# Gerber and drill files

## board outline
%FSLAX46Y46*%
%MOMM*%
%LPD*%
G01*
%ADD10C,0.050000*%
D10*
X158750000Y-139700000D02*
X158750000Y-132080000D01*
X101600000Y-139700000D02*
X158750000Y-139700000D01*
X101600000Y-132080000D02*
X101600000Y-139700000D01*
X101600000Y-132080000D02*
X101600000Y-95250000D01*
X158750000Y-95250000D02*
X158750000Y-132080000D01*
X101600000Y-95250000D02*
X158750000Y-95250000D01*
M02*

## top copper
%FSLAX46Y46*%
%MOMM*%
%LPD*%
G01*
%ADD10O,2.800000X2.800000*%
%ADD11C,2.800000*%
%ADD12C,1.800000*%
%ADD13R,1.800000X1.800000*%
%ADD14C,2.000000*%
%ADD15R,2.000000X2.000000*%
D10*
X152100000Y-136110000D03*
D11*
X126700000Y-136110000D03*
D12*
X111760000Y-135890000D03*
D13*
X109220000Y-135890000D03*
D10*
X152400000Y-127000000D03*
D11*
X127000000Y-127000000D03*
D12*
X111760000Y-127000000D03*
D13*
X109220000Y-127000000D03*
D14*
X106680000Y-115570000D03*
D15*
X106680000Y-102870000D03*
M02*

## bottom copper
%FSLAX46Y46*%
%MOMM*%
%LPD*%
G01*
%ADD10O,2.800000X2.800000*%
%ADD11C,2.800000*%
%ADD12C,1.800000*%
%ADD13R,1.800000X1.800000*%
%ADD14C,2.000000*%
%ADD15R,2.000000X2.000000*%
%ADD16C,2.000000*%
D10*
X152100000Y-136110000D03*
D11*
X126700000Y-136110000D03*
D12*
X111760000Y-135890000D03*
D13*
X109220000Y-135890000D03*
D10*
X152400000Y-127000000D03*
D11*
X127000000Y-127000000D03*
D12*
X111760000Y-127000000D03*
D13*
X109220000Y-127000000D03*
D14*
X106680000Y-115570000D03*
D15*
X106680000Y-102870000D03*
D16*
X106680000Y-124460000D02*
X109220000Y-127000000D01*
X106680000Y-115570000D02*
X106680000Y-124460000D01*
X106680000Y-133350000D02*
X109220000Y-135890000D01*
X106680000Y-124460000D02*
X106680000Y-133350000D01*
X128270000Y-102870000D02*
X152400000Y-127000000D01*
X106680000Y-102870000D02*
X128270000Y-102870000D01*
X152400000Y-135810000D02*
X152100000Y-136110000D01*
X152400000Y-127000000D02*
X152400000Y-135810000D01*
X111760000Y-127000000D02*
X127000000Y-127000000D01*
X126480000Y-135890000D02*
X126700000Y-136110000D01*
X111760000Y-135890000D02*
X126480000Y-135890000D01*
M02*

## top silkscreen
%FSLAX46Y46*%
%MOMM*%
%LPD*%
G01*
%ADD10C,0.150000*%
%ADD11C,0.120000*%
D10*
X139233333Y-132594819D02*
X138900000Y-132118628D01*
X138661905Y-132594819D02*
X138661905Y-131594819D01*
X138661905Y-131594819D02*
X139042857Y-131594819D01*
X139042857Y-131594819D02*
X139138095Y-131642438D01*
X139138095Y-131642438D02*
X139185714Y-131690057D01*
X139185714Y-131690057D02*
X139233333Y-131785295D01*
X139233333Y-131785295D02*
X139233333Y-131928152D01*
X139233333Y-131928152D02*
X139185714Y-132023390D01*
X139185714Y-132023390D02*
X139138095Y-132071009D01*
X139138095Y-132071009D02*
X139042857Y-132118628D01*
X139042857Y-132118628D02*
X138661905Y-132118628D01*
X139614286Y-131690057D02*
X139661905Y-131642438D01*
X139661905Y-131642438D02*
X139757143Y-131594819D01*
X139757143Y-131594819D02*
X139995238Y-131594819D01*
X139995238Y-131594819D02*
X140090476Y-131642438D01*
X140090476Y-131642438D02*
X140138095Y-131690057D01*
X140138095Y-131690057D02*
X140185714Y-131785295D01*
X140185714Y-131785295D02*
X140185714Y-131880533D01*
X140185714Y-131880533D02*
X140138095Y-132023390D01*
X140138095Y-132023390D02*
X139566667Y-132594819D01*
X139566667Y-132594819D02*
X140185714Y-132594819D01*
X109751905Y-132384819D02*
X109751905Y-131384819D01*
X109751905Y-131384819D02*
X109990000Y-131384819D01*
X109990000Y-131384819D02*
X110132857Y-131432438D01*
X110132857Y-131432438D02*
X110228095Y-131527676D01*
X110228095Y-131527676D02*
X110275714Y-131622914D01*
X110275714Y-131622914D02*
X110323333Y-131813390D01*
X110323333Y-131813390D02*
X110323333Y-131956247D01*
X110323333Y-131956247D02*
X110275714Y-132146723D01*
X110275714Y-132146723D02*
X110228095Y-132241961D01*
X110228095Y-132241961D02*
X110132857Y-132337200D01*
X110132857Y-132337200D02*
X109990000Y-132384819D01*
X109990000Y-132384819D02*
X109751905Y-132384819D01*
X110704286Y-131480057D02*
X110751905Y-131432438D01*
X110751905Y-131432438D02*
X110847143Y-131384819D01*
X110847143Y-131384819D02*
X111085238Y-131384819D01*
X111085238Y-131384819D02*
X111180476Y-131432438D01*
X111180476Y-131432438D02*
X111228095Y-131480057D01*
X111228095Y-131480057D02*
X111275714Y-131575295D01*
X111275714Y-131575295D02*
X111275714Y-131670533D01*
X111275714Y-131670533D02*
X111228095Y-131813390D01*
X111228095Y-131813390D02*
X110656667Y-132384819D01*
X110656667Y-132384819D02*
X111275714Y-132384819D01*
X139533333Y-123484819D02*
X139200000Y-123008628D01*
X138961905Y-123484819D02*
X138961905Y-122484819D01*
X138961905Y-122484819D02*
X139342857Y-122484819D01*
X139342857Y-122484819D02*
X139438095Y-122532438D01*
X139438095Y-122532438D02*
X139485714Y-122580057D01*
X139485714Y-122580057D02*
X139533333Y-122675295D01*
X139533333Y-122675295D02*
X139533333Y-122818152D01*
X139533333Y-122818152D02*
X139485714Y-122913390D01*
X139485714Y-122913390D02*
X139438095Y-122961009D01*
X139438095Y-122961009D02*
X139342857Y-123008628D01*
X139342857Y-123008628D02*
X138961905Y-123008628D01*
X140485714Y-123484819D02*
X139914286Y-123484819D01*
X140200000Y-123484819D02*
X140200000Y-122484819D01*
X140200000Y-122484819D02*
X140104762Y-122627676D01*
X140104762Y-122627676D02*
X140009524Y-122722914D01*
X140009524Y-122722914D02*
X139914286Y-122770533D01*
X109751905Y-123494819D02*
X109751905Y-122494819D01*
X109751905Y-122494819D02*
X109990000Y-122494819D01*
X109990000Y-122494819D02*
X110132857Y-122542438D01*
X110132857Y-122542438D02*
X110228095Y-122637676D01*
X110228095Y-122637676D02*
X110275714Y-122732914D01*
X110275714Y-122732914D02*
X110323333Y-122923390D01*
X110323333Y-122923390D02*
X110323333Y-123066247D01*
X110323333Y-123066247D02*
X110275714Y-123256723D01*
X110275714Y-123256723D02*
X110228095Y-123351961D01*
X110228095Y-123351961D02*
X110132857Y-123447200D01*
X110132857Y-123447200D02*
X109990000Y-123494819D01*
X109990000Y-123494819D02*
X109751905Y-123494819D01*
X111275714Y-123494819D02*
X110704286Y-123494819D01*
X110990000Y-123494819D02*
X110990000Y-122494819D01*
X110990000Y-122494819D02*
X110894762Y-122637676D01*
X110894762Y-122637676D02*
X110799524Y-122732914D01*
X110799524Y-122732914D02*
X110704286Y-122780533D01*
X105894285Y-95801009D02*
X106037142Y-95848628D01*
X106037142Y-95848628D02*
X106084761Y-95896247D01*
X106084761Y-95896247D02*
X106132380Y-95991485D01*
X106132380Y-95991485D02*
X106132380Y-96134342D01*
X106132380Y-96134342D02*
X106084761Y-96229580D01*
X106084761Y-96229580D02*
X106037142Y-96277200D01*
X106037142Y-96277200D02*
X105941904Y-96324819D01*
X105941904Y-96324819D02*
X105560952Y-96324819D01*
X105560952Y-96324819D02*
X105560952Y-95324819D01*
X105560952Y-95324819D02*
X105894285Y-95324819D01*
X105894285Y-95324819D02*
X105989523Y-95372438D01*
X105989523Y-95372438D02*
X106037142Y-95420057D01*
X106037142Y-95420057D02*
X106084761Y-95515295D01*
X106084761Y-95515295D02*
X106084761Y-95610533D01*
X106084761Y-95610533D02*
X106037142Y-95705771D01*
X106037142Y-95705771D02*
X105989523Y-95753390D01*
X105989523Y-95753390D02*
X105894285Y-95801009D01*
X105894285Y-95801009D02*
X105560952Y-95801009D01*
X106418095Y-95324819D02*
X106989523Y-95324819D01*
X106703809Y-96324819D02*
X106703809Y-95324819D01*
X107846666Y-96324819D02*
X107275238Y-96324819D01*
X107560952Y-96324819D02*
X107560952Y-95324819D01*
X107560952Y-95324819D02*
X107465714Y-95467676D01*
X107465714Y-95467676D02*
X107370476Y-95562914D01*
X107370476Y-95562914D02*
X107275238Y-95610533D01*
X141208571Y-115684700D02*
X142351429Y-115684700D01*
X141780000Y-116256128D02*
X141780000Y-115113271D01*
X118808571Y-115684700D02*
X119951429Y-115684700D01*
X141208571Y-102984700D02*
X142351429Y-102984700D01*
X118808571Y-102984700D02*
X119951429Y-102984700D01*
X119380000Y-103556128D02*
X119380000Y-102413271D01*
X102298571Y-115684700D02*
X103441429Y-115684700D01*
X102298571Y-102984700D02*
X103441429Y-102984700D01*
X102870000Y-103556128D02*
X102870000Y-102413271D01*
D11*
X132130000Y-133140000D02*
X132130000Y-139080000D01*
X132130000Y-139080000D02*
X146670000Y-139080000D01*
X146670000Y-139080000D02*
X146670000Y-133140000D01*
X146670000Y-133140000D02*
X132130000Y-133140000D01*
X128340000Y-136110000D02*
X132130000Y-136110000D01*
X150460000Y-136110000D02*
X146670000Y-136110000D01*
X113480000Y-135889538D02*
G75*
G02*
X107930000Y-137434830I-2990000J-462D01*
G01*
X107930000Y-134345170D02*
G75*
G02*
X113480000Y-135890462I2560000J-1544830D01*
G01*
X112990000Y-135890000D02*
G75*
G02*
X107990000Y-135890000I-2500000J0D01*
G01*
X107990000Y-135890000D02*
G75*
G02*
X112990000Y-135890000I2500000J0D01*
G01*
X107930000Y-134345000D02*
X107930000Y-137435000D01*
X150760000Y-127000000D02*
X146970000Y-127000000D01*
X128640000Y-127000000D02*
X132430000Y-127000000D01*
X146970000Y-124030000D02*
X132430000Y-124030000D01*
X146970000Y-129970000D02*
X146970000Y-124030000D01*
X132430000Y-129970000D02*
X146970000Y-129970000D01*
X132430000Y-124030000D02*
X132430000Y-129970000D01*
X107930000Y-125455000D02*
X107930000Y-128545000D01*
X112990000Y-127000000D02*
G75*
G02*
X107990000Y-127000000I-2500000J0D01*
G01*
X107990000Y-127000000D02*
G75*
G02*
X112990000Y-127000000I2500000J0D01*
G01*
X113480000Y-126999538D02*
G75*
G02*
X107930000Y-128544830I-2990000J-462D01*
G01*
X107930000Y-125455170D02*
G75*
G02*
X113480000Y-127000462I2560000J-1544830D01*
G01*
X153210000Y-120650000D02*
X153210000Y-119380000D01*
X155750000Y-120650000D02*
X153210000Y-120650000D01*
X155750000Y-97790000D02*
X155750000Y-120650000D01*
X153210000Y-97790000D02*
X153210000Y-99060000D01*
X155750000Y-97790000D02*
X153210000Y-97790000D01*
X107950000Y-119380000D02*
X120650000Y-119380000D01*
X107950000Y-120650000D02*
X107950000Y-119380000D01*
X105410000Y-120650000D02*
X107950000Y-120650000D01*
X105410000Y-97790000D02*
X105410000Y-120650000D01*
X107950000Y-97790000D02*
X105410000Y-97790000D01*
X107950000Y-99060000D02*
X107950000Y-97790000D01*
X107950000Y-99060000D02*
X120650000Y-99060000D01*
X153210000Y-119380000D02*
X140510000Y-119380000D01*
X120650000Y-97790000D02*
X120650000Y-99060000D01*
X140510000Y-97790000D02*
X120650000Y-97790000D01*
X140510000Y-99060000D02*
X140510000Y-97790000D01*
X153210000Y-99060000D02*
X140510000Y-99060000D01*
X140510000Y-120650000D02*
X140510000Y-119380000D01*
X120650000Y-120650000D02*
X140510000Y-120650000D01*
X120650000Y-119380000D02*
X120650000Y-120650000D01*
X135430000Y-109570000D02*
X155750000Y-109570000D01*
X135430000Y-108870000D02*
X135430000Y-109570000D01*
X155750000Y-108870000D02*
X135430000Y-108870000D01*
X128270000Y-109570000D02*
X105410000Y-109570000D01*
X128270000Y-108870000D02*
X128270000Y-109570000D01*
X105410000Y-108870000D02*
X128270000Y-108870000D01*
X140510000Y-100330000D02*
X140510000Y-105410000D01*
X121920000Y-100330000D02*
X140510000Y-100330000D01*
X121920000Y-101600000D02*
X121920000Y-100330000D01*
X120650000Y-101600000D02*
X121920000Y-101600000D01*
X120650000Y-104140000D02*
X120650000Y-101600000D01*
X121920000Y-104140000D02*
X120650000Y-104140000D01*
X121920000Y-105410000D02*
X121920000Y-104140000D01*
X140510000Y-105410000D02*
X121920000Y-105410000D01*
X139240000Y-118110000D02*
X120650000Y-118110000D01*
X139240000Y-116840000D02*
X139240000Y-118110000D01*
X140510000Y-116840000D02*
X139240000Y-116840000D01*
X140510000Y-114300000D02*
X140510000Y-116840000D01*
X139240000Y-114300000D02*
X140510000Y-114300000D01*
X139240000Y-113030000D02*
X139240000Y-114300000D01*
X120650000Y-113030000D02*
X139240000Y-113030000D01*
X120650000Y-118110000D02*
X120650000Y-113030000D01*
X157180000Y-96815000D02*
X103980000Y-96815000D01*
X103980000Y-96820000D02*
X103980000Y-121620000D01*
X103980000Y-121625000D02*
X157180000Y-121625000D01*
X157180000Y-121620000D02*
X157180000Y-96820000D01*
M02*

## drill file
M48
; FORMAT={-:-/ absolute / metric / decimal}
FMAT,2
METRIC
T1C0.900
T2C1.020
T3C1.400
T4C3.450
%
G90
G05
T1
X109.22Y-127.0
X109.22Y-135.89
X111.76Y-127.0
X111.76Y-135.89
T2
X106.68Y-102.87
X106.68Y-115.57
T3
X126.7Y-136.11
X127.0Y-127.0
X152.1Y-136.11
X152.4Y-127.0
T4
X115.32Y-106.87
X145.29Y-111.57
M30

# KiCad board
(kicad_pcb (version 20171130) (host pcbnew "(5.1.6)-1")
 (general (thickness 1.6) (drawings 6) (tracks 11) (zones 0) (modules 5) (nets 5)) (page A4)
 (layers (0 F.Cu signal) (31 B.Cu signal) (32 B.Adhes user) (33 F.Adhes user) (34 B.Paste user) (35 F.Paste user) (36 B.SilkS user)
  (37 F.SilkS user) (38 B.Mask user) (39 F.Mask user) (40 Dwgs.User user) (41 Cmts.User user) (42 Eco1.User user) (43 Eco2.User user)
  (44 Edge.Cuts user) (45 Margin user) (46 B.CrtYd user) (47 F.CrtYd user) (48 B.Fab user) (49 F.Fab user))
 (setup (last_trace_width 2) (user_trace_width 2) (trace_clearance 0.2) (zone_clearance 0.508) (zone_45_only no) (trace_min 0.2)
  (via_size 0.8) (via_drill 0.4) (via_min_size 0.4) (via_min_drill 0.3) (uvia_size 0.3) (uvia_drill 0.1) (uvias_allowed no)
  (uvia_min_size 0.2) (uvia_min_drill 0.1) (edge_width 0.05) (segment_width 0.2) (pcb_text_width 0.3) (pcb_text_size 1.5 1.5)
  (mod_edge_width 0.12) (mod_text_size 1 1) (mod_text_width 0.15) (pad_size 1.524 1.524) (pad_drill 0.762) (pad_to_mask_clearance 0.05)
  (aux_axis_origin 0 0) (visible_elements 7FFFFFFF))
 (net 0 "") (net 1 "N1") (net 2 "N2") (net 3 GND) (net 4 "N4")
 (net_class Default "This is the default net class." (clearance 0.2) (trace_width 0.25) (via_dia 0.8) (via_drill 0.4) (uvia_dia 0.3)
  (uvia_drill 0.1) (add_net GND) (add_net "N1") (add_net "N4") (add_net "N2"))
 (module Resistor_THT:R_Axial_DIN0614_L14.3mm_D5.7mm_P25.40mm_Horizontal (layer F.Cu) (at 126.7 136.11)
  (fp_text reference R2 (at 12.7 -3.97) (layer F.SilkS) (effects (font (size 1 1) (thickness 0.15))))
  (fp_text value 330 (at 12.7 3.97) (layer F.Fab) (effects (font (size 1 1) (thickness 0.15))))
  (fp_line (start 5.43 -2.97) (end 5.43 2.97) (layer F.SilkS) (width 0.12))
  (fp_line (start 5.43 2.97) (end 19.97 2.97) (layer F.SilkS) (width 0.12))
  (fp_line (start 19.97 2.97) (end 19.97 -2.97) (layer F.SilkS) (width 0.12))
  (fp_line (start 19.97 -2.97) (end 5.43 -2.97) (layer F.SilkS) (width 0.12))
  (fp_line (start 1.64 0) (end 5.43 0) (layer F.SilkS) (width 0.12))
  (fp_line (start 23.76 0) (end 19.97 0) (layer F.SilkS) (width 0.12))
  (pad 2 thru_hole oval (at 25.4 0) (size 2.8 2.8) (drill 1.4) (layers *.Cu *.Mask) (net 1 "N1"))
  (pad 1 thru_hole circle (at 0 0) (size 2.8 2.8) (drill 1.4) (layers *.Cu *.Mask) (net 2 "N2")))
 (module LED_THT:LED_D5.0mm (layer F.Cu) (at 109.22 135.89)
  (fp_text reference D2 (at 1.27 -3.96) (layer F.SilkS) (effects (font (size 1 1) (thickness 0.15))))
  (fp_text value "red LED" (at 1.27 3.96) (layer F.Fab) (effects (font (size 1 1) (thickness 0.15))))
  (fp_arc (start 1.27 0) (end -1.29 1.54483) (angle -148.9) (layer F.SilkS) (width 0.12))
  (fp_arc (start 1.27 0) (end -1.29 -1.54483) (angle 148.9) (layer F.SilkS) (width 0.12))
  (fp_circle (center 1.27 0) (end 3.77 0) (layer F.SilkS) (width 0.12))
  (fp_line (start -1.29 -1.545) (end -1.29 1.545) (layer F.SilkS) (width 0.12))
  (pad 2 thru_hole circle (at 2.54 0) (size 1.8 1.8) (drill 0.9) (layers *.Cu *.Mask) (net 2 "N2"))
  (pad 1 thru_hole rect (at 0 0) (size 1.8 1.8) (drill 0.9) (layers *.Cu *.Mask) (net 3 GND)))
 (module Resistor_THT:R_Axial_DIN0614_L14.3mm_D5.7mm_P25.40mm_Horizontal (layer F.Cu) (at 127 127)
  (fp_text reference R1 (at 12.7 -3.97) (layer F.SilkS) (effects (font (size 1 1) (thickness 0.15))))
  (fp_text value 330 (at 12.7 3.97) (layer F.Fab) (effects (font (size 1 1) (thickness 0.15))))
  (fp_line (start 23.76 0) (end 19.97 0) (layer F.SilkS) (width 0.12))
  (fp_line (start 1.64 0) (end 5.43 0) (layer F.SilkS) (width 0.12))
  (fp_line (start 19.97 -2.97) (end 5.43 -2.97) (layer F.SilkS) (width 0.12))
  (fp_line (start 19.97 2.97) (end 19.97 -2.97) (layer F.SilkS) (width 0.12))
  (fp_line (start 5.43 2.97) (end 19.97 2.97) (layer F.SilkS) (width 0.12))
  (fp_line (start 5.43 -2.97) (end 5.43 2.97) (layer F.SilkS) (width 0.12))
  (pad 2 thru_hole oval (at 25.4 0) (size 2.8 2.8) (drill 1.4) (layers *.Cu *.Mask) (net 1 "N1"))
  (pad 1 thru_hole circle (at 0 0) (size 2.8 2.8) (drill 1.4) (layers *.Cu *.Mask) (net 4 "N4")))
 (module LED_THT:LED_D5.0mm (layer F.Cu) (at 109.22 127)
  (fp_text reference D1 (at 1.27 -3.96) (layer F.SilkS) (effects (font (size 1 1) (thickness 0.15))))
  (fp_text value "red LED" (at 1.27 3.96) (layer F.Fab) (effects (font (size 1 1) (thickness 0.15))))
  (fp_line (start -1.29 -1.545) (end -1.29 1.545) (layer F.SilkS) (width 0.12))
  (fp_circle (center 1.27 0) (end 3.77 0) (layer F.SilkS) (width 0.12))
  (fp_arc (start 1.27 0) (end -1.29 1.54483) (angle -148.9) (layer F.SilkS) (width 0.12))
  (fp_arc (start 1.27 0) (end -1.29 -1.54483) (angle 148.9) (layer F.SilkS) (width 0.12))
  (pad 2 thru_hole circle (at 2.54 0) (size 1.8 1.8) (drill 0.9) (layers *.Cu *.Mask) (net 4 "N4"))
  (pad 1 thru_hole rect (at 0 0) (size 1.8 1.8) (drill 0.9) (layers *.Cu *.Mask) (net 3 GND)))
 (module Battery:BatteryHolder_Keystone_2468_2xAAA (layer F.Cu) (at 106.68 102.87)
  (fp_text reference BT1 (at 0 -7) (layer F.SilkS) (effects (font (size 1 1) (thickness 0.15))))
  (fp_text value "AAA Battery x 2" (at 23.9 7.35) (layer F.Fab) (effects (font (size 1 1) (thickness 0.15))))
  (fp_line (start 46.53 17.78) (end 46.53 16.51) (layer F.SilkS) (width 0.12))
  (fp_line (start 49.07 17.78) (end 46.53 17.78) (layer F.SilkS) (width 0.12))
  (fp_line (start 49.07 -5.08) (end 49.07 17.78) (layer F.SilkS) (width 0.12))
  (fp_line (start 46.53 -5.08) (end 46.53 -3.81) (layer F.SilkS) (width 0.12))
  (fp_line (start 49.07 -5.08) (end 46.53 -5.08) (layer F.SilkS) (width 0.12))
  (fp_line (start 1.27 16.51) (end 13.97 16.51) (layer F.SilkS) (width 0.12))
  (fp_line (start 1.27 17.78) (end 1.27 16.51) (layer F.SilkS) (width 0.12))
  (fp_line (start -1.27 17.78) (end 1.27 17.78) (layer F.SilkS) (width 0.12))
  (fp_line (start -1.27 -5.08) (end -1.27 17.78) (layer F.SilkS) (width 0.12))
  (fp_line (start 1.27 -5.08) (end -1.27 -5.08) (layer F.SilkS) (width 0.12))
  (fp_line (start 1.27 -3.81) (end 1.27 -5.08) (layer F.SilkS) (width 0.12))
  (fp_line (start 1.27 -3.81) (end 13.97 -3.81) (layer F.SilkS) (width 0.12))
  (fp_line (start 46.53 16.51) (end 33.83 16.51) (layer F.SilkS) (width 0.12))
  (fp_line (start 13.97 -5.08) (end 13.97 -3.81) (layer F.SilkS) (width 0.12))
  (fp_line (start 33.83 -5.08) (end 13.97 -5.08) (layer F.SilkS) (width 0.12))
  (fp_line (start 33.83 -3.81) (end 33.83 -5.08) (layer F.SilkS) (width 0.12))
  (fp_line (start 46.53 -3.81) (end 33.83 -3.81) (layer F.SilkS) (width 0.12))
  (fp_line (start 33.83 17.78) (end 33.83 16.51) (layer F.SilkS) (width 0.12))
  (fp_line (start 13.97 17.78) (end 33.83 17.78) (layer F.SilkS) (width 0.12))
  (fp_line (start 13.97 16.51) (end 13.97 17.78) (layer F.SilkS) (width 0.12))
  (fp_line (start 28.75 6.7) (end 49.07 6.7) (layer F.SilkS) (width 0.12))
  (fp_line (start 28.75 6) (end 28.75 6.7) (layer F.SilkS) (width 0.12))
  (fp_line (start 49.07 6) (end 28.75 6) (layer F.SilkS) (width 0.12))
  (fp_line (start 21.59 6.7) (end -1.27 6.7) (layer F.SilkS) (width 0.12))
  (fp_line (start 21.59 6) (end 21.59 6.7) (layer F.SilkS) (width 0.12))
  (fp_line (start -1.27 6) (end 21.59 6) (layer F.SilkS) (width 0.12))
  (fp_line (start 33.83 -2.54) (end 33.83 2.54) (layer F.SilkS) (width 0.12))
  (fp_line (start 15.24 -2.54) (end 33.83 -2.54) (layer F.SilkS) (width 0.12))
  (fp_line (start 15.24 -1.27) (end 15.24 -2.54) (layer F.SilkS) (width 0.12))
  (fp_line (start 13.97 -1.27) (end 15.24 -1.27) (layer F.SilkS) (width 0.12))
  (fp_line (start 13.97 1.27) (end 13.97 -1.27) (layer F.SilkS) (width 0.12))
  (fp_line (start 15.24 1.27) (end 13.97 1.27) (layer F.SilkS) (width 0.12))
  (fp_line (start 15.24 2.54) (end 15.24 1.27) (layer F.SilkS) (width 0.12))
  (fp_line (start 33.83 2.54) (end 15.24 2.54) (layer F.SilkS) (width 0.12))
  (fp_line (start 32.56 15.24) (end 13.97 15.24) (layer F.SilkS) (width 0.12))
  (fp_line (start 32.56 13.97) (end 32.56 15.24) (layer F.SilkS) (width 0.12))
  (fp_line (start 33.83 13.97) (end 32.56 13.97) (layer F.SilkS) (width 0.12))
  (fp_line (start 33.83 11.43) (end 33.83 13.97) (layer F.SilkS) (width 0.12))
  (fp_line (start 32.56 11.43) (end 33.83 11.43) (layer F.SilkS) (width 0.12))
  (fp_line (start 32.56 10.16) (end 32.56 11.43) (layer F.SilkS) (width 0.12))
  (fp_line (start 13.97 10.16) (end 32.56 10.16) (layer F.SilkS) (width 0.12))
  (fp_line (start 13.97 15.24) (end 13.97 10.16) (layer F.SilkS) (width 0.12))
  (fp_line (start 50.5 -6.055) (end -2.7 -6.055) (layer F.SilkS) (width 0.12))
  (fp_line (start -2.7 -6.05) (end -2.7 18.75) (layer F.SilkS) (width 0.12))
  (fp_line (start -2.7 18.755) (end 50.5 18.755) (layer F.SilkS) (width 0.12))
  (fp_line (start 50.5 18.75) (end 50.5 -6.05) (layer F.SilkS) (width 0.12))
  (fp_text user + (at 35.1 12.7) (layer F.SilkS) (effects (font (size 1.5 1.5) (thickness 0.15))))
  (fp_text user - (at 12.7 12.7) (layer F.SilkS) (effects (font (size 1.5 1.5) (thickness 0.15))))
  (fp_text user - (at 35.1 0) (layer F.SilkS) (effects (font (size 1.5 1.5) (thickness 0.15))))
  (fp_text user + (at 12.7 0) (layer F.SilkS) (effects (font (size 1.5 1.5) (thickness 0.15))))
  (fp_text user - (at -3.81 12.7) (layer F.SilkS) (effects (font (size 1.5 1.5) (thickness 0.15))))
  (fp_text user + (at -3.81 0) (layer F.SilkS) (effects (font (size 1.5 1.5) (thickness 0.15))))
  (pad "" np_thru_hole circle (at 38.61 8.7) (size 3.45 3.45) (drill 3.45) (layers *.Cu *.Mask))
  (pad "" np_thru_hole circle (at 8.64 4) (size 3.45 3.45) (drill 3.45) (layers *.Cu))
  (pad 2 thru_hole circle (at 0 12.7) (size 2 2) (drill 1.02) (layers *.Cu *.Mask) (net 3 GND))
  (pad 1 thru_hole rect (at 0 0) (size 2 2) (drill 1.02) (layers *.Cu *.Mask) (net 1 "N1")))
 (gr_line (start 158.75 139.7) (end 158.75 132.08) (layer Edge.Cuts) (width 0.05))
 (gr_line (start 101.6 139.7) (end 158.75 139.7) (layer Edge.Cuts) (width 0.05))
 (gr_line (start 101.6 132.08) (end 101.6 139.7) (layer Edge.Cuts) (width 0.05))
 (gr_line (start 101.6 132.08) (end 101.6 95.25) (layer Edge.Cuts) (width 0.05))
 (gr_line (start 158.75 95.25) (end 158.75 132.08) (layer Edge.Cuts) (width 0.05))
 (gr_line (start 101.6 95.25) (end 158.75 95.25) (layer Edge.Cuts) (width 0.05))
 (segment (start 106.68 124.46) (end 109.22 127) (width 2) (layer B.Cu) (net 3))
 (segment (start 106.68 115.57) (end 106.68 124.46) (width 2) (layer B.Cu) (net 3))
 (segment (start 106.68 133.35) (end 109.22 135.89) (width 2) (layer B.Cu) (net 3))
 (segment (start 106.68 124.46) (end 106.68 133.35) (width 2) (layer B.Cu) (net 3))
 (segment (start 128.27 102.87) (end 152.4 127) (width 2) (layer B.Cu) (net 1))
 (segment (start 106.68 102.87) (end 128.27 102.87) (width 2) (layer B.Cu) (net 1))
 (segment (start 152.4 135.81) (end 152.1 136.11) (width 2) (layer B.Cu) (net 1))
 (segment (start 152.4 127) (end 152.4 135.81) (width 2) (layer B.Cu) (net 1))
 (segment (start 111.76 127) (end 127 127) (width 2) (layer B.Cu) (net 4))
 (segment (start 126.48 135.89) (end 126.7 136.11) (width 2) (layer B.Cu) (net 2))
 (segment (start 111.76 135.89) (end 126.48 135.89) (width 2) (layer B.Cu) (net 2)))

